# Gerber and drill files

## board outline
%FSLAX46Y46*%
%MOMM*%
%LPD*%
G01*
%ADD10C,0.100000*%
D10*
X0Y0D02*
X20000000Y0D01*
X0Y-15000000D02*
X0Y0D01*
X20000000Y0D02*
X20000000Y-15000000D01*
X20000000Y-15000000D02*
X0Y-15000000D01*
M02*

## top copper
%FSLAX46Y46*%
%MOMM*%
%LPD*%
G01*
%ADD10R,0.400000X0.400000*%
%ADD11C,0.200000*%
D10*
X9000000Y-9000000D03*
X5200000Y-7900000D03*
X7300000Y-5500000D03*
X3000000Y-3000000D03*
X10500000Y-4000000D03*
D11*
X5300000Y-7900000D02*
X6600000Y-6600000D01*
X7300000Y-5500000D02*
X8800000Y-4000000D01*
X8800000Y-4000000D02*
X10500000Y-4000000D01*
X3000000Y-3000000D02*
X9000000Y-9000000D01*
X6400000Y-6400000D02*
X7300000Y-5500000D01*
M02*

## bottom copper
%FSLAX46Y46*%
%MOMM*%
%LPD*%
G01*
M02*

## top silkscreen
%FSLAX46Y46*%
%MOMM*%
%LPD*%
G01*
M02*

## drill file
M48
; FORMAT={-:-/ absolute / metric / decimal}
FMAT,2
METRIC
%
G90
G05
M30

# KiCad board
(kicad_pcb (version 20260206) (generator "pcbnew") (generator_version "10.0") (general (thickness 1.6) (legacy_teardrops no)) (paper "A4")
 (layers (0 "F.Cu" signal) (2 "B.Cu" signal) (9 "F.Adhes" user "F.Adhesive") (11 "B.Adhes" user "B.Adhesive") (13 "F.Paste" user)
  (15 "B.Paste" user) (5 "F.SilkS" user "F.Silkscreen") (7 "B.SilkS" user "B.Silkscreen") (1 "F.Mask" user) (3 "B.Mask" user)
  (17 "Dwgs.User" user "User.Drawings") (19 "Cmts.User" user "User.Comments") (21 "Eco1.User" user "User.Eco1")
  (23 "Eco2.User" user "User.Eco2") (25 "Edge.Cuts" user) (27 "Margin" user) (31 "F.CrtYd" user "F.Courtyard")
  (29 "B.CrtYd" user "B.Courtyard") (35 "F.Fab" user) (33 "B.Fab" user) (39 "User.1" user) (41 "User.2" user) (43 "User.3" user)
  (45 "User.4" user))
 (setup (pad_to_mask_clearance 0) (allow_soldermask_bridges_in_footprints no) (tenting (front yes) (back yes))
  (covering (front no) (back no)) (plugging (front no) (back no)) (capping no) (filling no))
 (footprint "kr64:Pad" (layer "F.Cu") (at 9 9)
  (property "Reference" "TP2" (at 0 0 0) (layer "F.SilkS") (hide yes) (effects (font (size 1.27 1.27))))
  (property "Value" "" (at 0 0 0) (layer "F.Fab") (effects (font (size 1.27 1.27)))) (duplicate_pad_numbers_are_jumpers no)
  (pad "1" smd rect (at 0 0) (size 0.4 0.4) (layers "F.Cu" "F.Mask" "F.Paste") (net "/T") (thermal_bridge_angle 45)))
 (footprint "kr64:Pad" (layer "F.Cu") (at 5.2 7.9)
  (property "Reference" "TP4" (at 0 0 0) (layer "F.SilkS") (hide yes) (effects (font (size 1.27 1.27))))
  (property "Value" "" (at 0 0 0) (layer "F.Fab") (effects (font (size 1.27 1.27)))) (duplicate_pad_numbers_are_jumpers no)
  (pad "1" smd rect (at 0 0) (size 0.4 0.4) (layers "F.Cu" "F.Mask" "F.Paste") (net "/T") (thermal_bridge_angle 45)))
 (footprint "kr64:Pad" (layer "F.Cu") (at 7.3 5.5)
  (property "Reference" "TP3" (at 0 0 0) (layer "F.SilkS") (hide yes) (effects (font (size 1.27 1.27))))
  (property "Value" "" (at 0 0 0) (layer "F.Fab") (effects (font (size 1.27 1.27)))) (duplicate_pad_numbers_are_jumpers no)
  (pad "1" smd rect (at 0 0) (size 0.4 0.4) (layers "F.Cu" "F.Mask" "F.Paste") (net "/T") (thermal_bridge_angle 45)))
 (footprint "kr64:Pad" (layer "F.Cu") (at 3 3)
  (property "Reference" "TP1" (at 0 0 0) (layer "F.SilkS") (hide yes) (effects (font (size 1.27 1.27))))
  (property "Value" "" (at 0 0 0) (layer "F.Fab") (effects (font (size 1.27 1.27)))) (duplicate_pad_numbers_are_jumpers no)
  (pad "1" smd rect (at 0 0) (size 0.4 0.4) (layers "F.Cu" "F.Mask" "F.Paste") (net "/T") (thermal_bridge_angle 45)))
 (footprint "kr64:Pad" (layer "F.Cu") (at 10.5 4)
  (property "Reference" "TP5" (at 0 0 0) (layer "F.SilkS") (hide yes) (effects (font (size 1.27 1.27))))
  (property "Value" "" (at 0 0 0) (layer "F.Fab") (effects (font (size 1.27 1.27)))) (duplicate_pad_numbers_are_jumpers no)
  (pad "1" smd rect (at 0 0) (size 0.4 0.4) (layers "F.Cu" "F.Mask" "F.Paste") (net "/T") (thermal_bridge_angle 45)))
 (gr_line (start 0 0) (end 20 0) (stroke (width 0.1) (type default)) (layer "Edge.Cuts"))
 (gr_line (start 0 15) (end 0 0) (stroke (width 0.1) (type default)) (layer "Edge.Cuts"))
 (gr_line (start 20 0) (end 20 15) (stroke (width 0.1) (type default)) (layer "Edge.Cuts"))
 (gr_line (start 20 15) (end 0 15) (stroke (width 0.1) (type default)) (layer "Edge.Cuts"))
 (segment (start 5.3 7.9) (end 6.6 6.6) (width 0.2) (layer "F.Cu") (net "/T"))
 (segment (start 7.3 5.5) (end 8.8 4) (width 0.2) (layer "F.Cu") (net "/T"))
 (segment (start 8.8 4) (end 10.5 4) (width 0.2) (layer "F.Cu") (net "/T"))
 (segment (start 3 3) (end 9 9) (width 0.2) (layer "F.Cu") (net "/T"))
 (segment (start 6.4 6.4) (end 7.3 5.5) (width 0.2) (layer "F.Cu") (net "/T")))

